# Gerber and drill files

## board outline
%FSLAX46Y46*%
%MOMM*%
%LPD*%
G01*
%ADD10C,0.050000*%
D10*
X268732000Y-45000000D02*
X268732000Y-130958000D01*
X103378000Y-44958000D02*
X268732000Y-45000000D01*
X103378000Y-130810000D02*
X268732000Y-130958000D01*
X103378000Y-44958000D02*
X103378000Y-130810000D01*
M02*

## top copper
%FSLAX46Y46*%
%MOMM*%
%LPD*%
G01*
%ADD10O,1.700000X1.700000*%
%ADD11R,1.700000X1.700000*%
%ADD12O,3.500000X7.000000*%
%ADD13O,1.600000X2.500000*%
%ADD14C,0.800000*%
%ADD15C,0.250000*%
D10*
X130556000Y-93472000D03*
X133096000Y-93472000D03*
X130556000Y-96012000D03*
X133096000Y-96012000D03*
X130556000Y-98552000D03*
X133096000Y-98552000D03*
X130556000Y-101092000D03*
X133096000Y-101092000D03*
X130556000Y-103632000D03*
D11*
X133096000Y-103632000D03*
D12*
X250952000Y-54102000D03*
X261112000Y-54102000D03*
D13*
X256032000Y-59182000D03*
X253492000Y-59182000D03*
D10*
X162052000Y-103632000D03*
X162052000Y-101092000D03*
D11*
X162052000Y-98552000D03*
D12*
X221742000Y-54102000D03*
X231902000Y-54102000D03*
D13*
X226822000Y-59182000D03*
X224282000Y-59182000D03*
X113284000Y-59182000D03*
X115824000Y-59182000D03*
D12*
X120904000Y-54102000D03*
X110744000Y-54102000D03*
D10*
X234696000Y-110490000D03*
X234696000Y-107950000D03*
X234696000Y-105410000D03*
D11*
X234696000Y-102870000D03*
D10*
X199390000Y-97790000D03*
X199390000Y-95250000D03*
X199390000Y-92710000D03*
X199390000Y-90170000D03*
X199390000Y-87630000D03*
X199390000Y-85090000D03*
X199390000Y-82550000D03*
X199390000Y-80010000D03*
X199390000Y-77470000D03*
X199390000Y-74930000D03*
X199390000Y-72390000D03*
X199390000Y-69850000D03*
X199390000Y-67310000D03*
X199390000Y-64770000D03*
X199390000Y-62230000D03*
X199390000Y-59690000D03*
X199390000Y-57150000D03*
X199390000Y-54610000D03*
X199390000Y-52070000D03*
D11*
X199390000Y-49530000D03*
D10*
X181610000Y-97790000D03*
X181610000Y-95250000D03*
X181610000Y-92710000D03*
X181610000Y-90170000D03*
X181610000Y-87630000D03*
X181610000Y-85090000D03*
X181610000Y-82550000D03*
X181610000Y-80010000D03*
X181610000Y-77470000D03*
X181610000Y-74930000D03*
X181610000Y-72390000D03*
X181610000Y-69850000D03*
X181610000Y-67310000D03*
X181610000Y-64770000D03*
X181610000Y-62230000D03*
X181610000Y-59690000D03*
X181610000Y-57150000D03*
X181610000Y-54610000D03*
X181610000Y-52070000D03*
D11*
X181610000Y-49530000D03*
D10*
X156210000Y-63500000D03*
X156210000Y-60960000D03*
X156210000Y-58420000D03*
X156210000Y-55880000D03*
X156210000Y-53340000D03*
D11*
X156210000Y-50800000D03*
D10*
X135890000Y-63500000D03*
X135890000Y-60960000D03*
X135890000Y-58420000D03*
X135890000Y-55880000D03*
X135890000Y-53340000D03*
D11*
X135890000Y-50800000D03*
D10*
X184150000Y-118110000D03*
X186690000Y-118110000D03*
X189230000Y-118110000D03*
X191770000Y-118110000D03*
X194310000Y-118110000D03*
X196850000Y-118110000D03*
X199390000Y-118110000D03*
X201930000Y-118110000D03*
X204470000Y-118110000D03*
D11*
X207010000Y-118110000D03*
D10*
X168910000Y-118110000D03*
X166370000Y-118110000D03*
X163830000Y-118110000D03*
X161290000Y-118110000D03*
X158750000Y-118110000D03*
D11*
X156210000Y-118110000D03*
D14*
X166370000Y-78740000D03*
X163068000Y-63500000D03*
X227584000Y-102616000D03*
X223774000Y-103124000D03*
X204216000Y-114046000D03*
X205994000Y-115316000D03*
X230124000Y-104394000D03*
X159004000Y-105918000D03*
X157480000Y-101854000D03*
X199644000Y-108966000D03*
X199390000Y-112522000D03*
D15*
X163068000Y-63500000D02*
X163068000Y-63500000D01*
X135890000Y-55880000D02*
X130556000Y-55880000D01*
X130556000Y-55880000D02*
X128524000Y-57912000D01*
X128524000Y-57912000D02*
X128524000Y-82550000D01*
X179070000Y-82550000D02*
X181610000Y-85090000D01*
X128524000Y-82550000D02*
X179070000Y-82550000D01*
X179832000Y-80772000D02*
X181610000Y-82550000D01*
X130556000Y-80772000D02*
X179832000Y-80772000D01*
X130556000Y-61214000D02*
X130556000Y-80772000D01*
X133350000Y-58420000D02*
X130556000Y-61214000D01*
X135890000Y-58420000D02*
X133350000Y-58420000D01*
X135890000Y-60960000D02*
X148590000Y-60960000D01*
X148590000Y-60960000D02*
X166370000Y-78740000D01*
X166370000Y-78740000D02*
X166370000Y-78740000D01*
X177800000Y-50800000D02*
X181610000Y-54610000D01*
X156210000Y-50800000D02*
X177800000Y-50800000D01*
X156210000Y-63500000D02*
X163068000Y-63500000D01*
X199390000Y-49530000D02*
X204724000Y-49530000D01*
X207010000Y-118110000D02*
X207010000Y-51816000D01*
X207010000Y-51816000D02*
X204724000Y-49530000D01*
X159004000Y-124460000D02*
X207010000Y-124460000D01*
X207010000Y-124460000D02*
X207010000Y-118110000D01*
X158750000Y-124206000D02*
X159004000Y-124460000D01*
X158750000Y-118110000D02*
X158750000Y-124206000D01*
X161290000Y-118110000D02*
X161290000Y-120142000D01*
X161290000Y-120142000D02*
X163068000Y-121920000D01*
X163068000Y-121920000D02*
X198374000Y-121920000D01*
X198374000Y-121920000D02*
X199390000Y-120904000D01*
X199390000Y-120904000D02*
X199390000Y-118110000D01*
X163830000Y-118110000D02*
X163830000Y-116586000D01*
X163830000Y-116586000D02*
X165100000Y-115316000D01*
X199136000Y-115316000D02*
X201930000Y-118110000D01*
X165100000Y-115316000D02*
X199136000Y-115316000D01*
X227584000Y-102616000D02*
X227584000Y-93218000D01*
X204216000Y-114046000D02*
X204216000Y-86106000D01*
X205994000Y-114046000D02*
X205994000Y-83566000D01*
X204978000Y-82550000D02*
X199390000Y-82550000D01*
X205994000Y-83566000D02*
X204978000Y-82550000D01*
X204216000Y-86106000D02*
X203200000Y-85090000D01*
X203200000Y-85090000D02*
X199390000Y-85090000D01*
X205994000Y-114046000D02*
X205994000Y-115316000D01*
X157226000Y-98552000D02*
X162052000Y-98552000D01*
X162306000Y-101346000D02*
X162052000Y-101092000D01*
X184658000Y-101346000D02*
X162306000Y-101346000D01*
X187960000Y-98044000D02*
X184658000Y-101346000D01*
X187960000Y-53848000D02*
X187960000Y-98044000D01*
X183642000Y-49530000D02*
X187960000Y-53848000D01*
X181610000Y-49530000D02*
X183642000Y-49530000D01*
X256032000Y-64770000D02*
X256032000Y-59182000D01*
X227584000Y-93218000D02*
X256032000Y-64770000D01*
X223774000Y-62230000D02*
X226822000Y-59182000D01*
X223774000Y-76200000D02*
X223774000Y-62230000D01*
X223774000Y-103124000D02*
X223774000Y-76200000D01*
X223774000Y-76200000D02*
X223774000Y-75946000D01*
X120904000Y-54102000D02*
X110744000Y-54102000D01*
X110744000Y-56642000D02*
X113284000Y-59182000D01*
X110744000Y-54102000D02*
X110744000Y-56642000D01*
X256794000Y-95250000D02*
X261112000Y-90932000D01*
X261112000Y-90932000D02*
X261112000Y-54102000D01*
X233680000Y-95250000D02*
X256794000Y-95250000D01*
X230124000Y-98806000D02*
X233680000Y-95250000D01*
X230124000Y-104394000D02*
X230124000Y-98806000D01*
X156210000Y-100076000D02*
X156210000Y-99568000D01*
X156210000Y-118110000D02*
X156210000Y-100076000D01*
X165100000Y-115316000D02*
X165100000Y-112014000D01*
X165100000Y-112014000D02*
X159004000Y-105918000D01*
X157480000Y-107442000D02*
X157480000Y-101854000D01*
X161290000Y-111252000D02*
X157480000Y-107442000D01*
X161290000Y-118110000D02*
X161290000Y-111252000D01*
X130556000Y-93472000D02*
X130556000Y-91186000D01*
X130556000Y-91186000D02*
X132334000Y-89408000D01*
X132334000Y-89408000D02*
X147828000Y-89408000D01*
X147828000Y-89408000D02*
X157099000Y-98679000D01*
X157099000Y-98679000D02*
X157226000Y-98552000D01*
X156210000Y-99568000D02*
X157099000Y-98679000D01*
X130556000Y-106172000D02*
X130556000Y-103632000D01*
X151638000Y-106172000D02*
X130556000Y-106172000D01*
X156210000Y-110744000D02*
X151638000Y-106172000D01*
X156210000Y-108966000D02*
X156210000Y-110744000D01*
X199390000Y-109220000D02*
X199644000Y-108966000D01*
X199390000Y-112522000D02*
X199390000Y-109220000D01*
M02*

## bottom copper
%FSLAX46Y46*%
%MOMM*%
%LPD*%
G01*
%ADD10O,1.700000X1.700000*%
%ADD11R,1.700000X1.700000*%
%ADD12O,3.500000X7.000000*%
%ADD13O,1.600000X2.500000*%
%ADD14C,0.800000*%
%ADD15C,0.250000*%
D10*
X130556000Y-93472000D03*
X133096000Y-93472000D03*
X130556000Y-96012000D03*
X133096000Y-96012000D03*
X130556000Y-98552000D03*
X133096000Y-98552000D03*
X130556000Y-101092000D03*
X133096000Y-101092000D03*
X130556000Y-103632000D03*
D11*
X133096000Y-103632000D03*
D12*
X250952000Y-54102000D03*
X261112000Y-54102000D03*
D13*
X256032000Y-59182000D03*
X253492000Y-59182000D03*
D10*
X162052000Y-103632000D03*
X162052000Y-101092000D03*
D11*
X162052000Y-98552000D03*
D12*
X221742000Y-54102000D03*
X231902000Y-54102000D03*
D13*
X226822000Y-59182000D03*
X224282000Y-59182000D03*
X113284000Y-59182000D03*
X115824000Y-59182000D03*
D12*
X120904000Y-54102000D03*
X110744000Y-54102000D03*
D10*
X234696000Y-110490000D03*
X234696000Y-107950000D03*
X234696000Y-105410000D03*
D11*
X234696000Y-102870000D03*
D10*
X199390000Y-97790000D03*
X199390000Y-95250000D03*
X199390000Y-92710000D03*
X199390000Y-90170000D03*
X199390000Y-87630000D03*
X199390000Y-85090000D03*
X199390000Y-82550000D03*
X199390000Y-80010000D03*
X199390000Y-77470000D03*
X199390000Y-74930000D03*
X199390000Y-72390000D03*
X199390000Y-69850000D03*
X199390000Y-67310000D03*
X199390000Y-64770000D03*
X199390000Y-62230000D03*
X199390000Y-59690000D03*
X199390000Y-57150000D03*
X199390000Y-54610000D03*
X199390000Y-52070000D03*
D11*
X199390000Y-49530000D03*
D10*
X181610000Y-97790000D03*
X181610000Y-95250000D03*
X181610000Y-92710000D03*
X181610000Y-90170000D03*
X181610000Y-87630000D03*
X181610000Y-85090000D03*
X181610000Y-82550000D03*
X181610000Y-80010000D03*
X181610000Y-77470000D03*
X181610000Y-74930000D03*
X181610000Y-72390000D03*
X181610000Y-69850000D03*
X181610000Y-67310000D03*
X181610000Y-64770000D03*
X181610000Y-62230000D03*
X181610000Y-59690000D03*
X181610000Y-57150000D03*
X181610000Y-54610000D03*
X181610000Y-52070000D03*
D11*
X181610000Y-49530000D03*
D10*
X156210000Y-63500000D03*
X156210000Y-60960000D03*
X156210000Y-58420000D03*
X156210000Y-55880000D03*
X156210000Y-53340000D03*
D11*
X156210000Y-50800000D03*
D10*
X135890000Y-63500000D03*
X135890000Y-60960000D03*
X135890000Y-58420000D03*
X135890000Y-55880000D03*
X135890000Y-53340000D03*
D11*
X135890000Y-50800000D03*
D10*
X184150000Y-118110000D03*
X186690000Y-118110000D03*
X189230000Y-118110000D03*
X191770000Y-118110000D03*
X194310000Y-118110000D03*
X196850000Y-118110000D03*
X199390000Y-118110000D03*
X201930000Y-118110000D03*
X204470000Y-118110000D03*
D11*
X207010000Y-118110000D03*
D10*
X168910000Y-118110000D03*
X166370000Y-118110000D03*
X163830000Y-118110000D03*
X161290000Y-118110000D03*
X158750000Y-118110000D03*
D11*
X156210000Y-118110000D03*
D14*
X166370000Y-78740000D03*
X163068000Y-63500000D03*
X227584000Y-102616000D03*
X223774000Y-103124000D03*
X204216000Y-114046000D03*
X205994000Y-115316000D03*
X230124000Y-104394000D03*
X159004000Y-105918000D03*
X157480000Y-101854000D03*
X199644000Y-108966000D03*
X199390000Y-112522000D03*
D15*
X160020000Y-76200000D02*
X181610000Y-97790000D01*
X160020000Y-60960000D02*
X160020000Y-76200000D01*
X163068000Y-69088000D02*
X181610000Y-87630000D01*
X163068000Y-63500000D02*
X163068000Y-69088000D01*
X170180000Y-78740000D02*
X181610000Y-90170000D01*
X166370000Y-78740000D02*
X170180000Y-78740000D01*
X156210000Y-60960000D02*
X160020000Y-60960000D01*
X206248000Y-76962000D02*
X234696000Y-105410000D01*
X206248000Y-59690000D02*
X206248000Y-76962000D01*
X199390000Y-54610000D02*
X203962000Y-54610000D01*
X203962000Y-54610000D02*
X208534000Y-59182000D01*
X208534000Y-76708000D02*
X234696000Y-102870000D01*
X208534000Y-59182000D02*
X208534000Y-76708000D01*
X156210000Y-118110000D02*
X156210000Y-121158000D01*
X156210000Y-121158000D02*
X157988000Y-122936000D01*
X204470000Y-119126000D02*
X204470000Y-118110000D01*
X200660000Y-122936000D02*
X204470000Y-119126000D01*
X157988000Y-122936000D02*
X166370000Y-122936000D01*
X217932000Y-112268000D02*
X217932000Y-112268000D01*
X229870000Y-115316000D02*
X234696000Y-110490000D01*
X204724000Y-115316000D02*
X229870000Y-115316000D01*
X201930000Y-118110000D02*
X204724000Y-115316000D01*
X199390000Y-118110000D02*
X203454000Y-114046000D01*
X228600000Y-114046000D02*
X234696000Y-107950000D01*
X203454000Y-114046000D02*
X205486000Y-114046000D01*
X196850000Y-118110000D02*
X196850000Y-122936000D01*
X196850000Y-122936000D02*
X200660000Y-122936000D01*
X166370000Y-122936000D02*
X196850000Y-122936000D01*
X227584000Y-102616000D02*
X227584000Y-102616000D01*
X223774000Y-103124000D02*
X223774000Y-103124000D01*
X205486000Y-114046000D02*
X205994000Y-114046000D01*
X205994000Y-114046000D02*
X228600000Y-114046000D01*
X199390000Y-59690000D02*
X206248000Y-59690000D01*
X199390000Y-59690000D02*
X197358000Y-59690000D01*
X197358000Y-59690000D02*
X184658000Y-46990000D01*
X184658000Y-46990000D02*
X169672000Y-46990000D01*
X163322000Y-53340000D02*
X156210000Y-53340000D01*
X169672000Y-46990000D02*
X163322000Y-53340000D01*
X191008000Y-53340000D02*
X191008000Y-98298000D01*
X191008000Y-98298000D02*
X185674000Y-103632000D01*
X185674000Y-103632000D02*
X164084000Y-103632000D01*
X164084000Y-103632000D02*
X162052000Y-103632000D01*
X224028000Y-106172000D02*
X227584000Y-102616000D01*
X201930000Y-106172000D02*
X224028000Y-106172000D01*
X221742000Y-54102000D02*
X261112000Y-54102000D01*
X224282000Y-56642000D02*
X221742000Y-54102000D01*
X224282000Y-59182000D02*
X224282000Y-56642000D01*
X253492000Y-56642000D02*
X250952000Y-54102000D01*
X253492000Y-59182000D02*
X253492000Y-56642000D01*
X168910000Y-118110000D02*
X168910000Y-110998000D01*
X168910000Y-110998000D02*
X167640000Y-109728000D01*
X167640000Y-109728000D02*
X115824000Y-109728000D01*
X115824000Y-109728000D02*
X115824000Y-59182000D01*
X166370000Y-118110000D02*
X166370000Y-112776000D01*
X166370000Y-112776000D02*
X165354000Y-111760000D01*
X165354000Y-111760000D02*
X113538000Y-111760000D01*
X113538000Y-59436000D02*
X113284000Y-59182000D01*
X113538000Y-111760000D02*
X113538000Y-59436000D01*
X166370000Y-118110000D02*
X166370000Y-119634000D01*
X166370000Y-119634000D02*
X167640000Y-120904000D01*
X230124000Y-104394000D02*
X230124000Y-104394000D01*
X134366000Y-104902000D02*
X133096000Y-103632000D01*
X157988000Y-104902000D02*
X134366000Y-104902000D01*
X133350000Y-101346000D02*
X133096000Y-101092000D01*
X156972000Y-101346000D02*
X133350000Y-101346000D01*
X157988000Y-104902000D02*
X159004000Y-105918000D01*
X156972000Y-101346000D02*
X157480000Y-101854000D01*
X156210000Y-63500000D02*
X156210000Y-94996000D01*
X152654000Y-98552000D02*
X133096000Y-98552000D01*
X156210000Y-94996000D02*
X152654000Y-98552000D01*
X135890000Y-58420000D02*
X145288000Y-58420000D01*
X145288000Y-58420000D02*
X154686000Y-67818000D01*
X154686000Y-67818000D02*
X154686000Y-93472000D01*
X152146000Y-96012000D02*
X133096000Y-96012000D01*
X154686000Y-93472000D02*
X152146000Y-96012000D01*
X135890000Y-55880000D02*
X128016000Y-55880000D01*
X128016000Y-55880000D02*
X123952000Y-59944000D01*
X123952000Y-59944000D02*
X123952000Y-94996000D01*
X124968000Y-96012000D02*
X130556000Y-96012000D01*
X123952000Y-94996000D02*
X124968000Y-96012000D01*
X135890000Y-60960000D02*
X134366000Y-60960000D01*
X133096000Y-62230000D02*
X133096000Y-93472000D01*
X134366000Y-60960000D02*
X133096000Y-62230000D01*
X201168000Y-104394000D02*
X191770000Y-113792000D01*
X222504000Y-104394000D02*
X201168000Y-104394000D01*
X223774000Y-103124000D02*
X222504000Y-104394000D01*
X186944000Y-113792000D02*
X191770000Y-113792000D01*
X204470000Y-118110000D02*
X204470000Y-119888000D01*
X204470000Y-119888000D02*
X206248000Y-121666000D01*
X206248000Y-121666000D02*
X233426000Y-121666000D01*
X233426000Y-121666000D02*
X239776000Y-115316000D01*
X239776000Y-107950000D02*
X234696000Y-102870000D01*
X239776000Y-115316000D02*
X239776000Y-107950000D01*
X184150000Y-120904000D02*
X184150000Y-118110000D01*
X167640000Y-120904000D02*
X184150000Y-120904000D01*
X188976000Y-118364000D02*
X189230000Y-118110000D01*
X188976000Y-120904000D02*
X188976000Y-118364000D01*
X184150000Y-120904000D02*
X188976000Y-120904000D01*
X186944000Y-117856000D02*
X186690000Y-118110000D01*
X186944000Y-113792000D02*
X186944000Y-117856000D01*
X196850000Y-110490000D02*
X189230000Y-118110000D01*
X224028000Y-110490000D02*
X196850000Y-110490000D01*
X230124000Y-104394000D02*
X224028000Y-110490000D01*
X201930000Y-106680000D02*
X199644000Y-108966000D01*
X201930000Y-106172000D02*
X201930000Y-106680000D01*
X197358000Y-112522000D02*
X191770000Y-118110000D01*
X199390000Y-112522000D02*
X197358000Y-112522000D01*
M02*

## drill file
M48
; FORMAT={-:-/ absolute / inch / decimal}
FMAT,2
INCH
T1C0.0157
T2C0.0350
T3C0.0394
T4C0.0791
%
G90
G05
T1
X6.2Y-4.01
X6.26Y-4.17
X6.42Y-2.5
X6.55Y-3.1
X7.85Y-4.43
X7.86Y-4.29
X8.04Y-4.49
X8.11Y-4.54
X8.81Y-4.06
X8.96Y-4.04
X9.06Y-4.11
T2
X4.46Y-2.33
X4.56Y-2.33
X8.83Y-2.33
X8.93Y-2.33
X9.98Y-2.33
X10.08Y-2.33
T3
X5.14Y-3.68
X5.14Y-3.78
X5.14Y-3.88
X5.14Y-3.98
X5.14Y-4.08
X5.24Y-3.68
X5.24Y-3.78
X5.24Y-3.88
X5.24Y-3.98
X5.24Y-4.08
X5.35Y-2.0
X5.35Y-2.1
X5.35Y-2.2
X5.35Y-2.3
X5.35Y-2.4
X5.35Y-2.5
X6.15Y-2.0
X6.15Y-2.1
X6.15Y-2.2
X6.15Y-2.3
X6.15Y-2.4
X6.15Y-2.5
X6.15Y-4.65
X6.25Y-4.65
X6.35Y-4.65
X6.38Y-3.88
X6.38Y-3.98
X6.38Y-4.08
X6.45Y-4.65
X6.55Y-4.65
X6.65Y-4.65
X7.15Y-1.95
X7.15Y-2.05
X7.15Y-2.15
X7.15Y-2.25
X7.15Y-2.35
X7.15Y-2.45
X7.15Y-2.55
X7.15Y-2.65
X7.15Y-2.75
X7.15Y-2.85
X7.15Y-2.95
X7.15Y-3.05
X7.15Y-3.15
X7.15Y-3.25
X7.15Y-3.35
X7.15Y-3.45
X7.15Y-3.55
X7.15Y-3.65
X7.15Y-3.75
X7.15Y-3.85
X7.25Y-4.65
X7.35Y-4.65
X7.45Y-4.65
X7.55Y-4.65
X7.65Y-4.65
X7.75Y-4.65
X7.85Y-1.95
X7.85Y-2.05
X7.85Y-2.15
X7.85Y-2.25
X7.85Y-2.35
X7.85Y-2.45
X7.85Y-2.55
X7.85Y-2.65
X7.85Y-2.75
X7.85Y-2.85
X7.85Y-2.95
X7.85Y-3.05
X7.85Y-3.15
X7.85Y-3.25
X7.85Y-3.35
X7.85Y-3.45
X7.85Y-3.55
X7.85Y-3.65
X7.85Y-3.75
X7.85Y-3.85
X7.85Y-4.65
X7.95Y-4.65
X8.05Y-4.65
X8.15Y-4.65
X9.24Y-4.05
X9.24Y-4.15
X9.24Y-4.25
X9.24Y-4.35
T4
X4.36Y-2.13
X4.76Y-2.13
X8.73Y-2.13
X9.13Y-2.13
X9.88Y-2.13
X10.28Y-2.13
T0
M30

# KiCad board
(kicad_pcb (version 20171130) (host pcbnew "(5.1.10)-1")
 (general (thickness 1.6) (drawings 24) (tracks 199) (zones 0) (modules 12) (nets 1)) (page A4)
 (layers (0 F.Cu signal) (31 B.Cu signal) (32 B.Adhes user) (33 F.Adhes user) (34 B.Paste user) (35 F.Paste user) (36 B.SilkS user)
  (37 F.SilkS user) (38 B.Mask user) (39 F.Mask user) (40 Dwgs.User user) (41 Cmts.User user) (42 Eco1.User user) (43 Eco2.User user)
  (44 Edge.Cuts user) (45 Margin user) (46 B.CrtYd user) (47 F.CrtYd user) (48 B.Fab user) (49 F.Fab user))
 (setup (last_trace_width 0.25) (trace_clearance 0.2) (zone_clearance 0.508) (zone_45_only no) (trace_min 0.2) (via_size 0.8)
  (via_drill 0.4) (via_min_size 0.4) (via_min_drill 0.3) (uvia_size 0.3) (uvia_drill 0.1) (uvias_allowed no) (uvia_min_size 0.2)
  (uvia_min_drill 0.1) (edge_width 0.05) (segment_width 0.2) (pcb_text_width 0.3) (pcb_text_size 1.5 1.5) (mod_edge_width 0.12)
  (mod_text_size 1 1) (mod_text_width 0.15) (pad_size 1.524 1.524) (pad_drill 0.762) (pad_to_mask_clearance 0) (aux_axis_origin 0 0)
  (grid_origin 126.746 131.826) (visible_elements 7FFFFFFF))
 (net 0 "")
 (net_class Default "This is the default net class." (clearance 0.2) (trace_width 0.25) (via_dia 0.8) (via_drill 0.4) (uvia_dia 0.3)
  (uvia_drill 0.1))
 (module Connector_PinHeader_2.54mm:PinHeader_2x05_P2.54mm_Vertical (layer F.Cu) (at 133.096 103.632 180)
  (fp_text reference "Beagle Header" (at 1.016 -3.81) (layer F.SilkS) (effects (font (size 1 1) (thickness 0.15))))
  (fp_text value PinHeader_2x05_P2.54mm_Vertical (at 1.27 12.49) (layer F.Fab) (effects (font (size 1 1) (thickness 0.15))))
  (pad 10 thru_hole oval (at 2.54 10.16 180) (size 1.7 1.7) (drill 1) (layers *.Cu *.Mask))
  (pad 9 thru_hole oval (at 0 10.16 180) (size 1.7 1.7) (drill 1) (layers *.Cu *.Mask))
  (pad 8 thru_hole oval (at 2.54 7.62 180) (size 1.7 1.7) (drill 1) (layers *.Cu *.Mask))
  (pad 7 thru_hole oval (at 0 7.62 180) (size 1.7 1.7) (drill 1) (layers *.Cu *.Mask))
  (pad 6 thru_hole oval (at 2.54 5.08 180) (size 1.7 1.7) (drill 1) (layers *.Cu *.Mask))
  (pad 5 thru_hole oval (at 0 5.08 180) (size 1.7 1.7) (drill 1) (layers *.Cu *.Mask))
  (pad 4 thru_hole oval (at 2.54 2.54 180) (size 1.7 1.7) (drill 1) (layers *.Cu *.Mask))
  (pad 3 thru_hole oval (at 0 2.54 180) (size 1.7 1.7) (drill 1) (layers *.Cu *.Mask))
  (pad 2 thru_hole oval (at 2.54 0 180) (size 1.7 1.7) (drill 1) (layers *.Cu *.Mask))
  (pad 1 thru_hole rect (at 0 0 180) (size 1.7 1.7) (drill 1) (layers *.Cu *.Mask)))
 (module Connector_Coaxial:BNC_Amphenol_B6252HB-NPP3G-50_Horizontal (layer F.Cu) (at 256.032 59.182)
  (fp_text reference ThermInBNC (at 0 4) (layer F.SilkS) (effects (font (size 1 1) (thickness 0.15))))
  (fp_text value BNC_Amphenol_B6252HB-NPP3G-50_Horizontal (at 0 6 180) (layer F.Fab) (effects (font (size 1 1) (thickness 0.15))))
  (pad 2 thru_hole oval (at -5.08 -5.08) (size 3.5 7) (drill 2.01) (layers *.Cu *.Mask))
  (pad 2 thru_hole oval (at 5.08 -5.08) (size 3.5 7) (drill 2.01) (layers *.Cu *.Mask))
  (pad 1 thru_hole oval (at 0 0) (size 1.6 2.5) (drill 0.89) (layers *.Cu *.Mask))
  (pad 2 thru_hole oval (at -2.54 0) (size 1.6 2.5) (drill 0.89) (layers *.Cu *.Mask)))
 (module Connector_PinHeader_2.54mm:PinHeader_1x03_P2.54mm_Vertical (layer F.Cu) (at 162.052 98.552)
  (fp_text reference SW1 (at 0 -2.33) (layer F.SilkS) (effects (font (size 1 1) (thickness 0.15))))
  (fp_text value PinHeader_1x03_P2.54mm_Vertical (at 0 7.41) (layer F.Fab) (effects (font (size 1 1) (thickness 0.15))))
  (pad 3 thru_hole oval (at 0 5.08) (size 1.7 1.7) (drill 1) (layers *.Cu *.Mask))
  (pad 2 thru_hole oval (at 0 2.54) (size 1.7 1.7) (drill 1) (layers *.Cu *.Mask))
  (pad 1 thru_hole rect (at 0 0) (size 1.7 1.7) (drill 1) (layers *.Cu *.Mask)))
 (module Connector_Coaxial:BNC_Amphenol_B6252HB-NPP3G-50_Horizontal (layer F.Cu) (at 226.822 59.182)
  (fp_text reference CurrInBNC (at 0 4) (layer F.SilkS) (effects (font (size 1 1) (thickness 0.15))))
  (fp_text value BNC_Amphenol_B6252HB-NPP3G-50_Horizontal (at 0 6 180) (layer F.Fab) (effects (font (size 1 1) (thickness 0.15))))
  (pad 2 thru_hole oval (at -5.08 -5.08) (size 3.5 7) (drill 2.01) (layers *.Cu *.Mask))
  (pad 2 thru_hole oval (at 5.08 -5.08) (size 3.5 7) (drill 2.01) (layers *.Cu *.Mask))
  (pad 1 thru_hole oval (at 0 0) (size 1.6 2.5) (drill 0.89) (layers *.Cu *.Mask))
  (pad 2 thru_hole oval (at -2.54 0) (size 1.6 2.5) (drill 0.89) (layers *.Cu *.Mask)))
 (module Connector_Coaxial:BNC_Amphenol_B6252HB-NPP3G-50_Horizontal (layer F.Cu) (at 115.824 59.182)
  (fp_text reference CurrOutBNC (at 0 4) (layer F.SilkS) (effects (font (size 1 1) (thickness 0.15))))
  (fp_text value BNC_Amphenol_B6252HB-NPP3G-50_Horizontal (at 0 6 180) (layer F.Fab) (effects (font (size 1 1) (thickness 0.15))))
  (pad 2 thru_hole oval (at -2.54 0) (size 1.6 2.5) (drill 0.89) (layers *.Cu *.Mask))
  (pad 1 thru_hole oval (at 0 0) (size 1.6 2.5) (drill 0.89) (layers *.Cu *.Mask))
  (pad 2 thru_hole oval (at 5.08 -5.08) (size 3.5 7) (drill 2.01) (layers *.Cu *.Mask))
  (pad 2 thru_hole oval (at -5.08 -5.08) (size 3.5 7) (drill 2.01) (layers *.Cu *.Mask)))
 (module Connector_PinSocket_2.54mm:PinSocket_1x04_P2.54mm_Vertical (layer F.Cu) (at 234.696 102.87)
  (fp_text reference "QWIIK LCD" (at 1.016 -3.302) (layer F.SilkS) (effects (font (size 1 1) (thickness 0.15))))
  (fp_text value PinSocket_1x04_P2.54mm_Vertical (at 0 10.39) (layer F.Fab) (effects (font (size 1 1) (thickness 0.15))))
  (pad 4 thru_hole oval (at 0 7.62) (size 1.7 1.7) (drill 1) (layers *.Cu *.Mask))
  (pad 3 thru_hole oval (at 0 5.08) (size 1.7 1.7) (drill 1) (layers *.Cu *.Mask))
  (pad 2 thru_hole oval (at 0 2.54) (size 1.7 1.7) (drill 1) (layers *.Cu *.Mask))
  (pad 1 thru_hole rect (at 0 0) (size 1.7 1.7) (drill 1) (layers *.Cu *.Mask)))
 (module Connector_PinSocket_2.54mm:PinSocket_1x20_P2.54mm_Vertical (layer F.Cu) (at 199.39 49.53)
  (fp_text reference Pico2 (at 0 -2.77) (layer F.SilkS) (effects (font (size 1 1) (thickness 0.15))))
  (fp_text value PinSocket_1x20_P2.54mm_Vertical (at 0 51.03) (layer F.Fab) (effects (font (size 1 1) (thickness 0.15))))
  (pad 20 thru_hole oval (at 0 48.26) (size 1.7 1.7) (drill 1) (layers *.Cu *.Mask))
  (pad 19 thru_hole oval (at 0 45.72) (size 1.7 1.7) (drill 1) (layers *.Cu *.Mask))
  (pad 18 thru_hole oval (at 0 43.18) (size 1.7 1.7) (drill 1) (layers *.Cu *.Mask))
  (pad 17 thru_hole oval (at 0 40.64) (size 1.7 1.7) (drill 1) (layers *.Cu *.Mask))
  (pad 16 thru_hole oval (at 0 38.1) (size 1.7 1.7) (drill 1) (layers *.Cu *.Mask))
  (pad 15 thru_hole oval (at 0 35.56) (size 1.7 1.7) (drill 1) (layers *.Cu *.Mask))
  (pad 14 thru_hole oval (at 0 33.02) (size 1.7 1.7) (drill 1) (layers *.Cu *.Mask))
  (pad 13 thru_hole oval (at 0 30.48) (size 1.7 1.7) (drill 1) (layers *.Cu *.Mask))
  (pad 12 thru_hole oval (at 0 27.94) (size 1.7 1.7) (drill 1) (layers *.Cu *.Mask))
  (pad 11 thru_hole oval (at 0 25.4) (size 1.7 1.7) (drill 1) (layers *.Cu *.Mask))
  (pad 10 thru_hole oval (at 0 22.86) (size 1.7 1.7) (drill 1) (layers *.Cu *.Mask))
  (pad 9 thru_hole oval (at 0 20.32) (size 1.7 1.7) (drill 1) (layers *.Cu *.Mask))
  (pad 8 thru_hole oval (at 0 17.78) (size 1.7 1.7) (drill 1) (layers *.Cu *.Mask))
  (pad 7 thru_hole oval (at 0 15.24) (size 1.7 1.7) (drill 1) (layers *.Cu *.Mask))
  (pad 6 thru_hole oval (at 0 12.7) (size 1.7 1.7) (drill 1) (layers *.Cu *.Mask))
  (pad 5 thru_hole oval (at 0 10.16) (size 1.7 1.7) (drill 1) (layers *.Cu *.Mask))
  (pad 4 thru_hole oval (at 0 7.62) (size 1.7 1.7) (drill 1) (layers *.Cu *.Mask))
  (pad 3 thru_hole oval (at 0 5.08) (size 1.7 1.7) (drill 1) (layers *.Cu *.Mask))
  (pad 2 thru_hole oval (at 0 2.54) (size 1.7 1.7) (drill 1) (layers *.Cu *.Mask))
  (pad 1 thru_hole rect (at 0 0) (size 1.7 1.7) (drill 1) (layers *.Cu *.Mask)))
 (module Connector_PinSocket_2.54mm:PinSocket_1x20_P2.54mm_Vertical (layer F.Cu) (at 181.61 49.53)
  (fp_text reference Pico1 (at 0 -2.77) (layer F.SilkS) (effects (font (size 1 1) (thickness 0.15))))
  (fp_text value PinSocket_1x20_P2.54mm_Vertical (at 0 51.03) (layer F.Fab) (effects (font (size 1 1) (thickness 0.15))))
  (pad 20 thru_hole oval (at 0 48.26) (size 1.7 1.7) (drill 1) (layers *.Cu *.Mask))
  (pad 19 thru_hole oval (at 0 45.72) (size 1.7 1.7) (drill 1) (layers *.Cu *.Mask))
  (pad 18 thru_hole oval (at 0 43.18) (size 1.7 1.7) (drill 1) (layers *.Cu *.Mask))
  (pad 17 thru_hole oval (at 0 40.64) (size 1.7 1.7) (drill 1) (layers *.Cu *.Mask))
  (pad 16 thru_hole oval (at 0 38.1) (size 1.7 1.7) (drill 1) (layers *.Cu *.Mask))
  (pad 15 thru_hole oval (at 0 35.56) (size 1.7 1.7) (drill 1) (layers *.Cu *.Mask))
  (pad 14 thru_hole oval (at 0 33.02) (size 1.7 1.7) (drill 1) (layers *.Cu *.Mask))
  (pad 13 thru_hole oval (at 0 30.48) (size 1.7 1.7) (drill 1) (layers *.Cu *.Mask))
  (pad 12 thru_hole oval (at 0 27.94) (size 1.7 1.7) (drill 1) (layers *.Cu *.Mask))
  (pad 11 thru_hole oval (at 0 25.4) (size 1.7 1.7) (drill 1) (layers *.Cu *.Mask))
  (pad 10 thru_hole oval (at 0 22.86) (size 1.7 1.7) (drill 1) (layers *.Cu *.Mask))
  (pad 9 thru_hole oval (at 0 20.32) (size 1.7 1.7) (drill 1) (layers *.Cu *.Mask))
  (pad 8 thru_hole oval (at 0 17.78) (size 1.7 1.7) (drill 1) (layers *.Cu *.Mask))
  (pad 7 thru_hole oval (at 0 15.24) (size 1.7 1.7) (drill 1) (layers *.Cu *.Mask))
  (pad 6 thru_hole oval (at 0 12.7) (size 1.7 1.7) (drill 1) (layers *.Cu *.Mask))
  (pad 5 thru_hole oval (at 0 10.16) (size 1.7 1.7) (drill 1) (layers *.Cu *.Mask))
  (pad 4 thru_hole oval (at 0 7.62) (size 1.7 1.7) (drill 1) (layers *.Cu *.Mask))
  (pad 3 thru_hole oval (at 0 5.08) (size 1.7 1.7) (drill 1) (layers *.Cu *.Mask))
  (pad 2 thru_hole oval (at 0 2.54) (size 1.7 1.7) (drill 1) (layers *.Cu *.Mask))
  (pad 1 thru_hole rect (at 0 0) (size 1.7 1.7) (drill 1) (layers *.Cu *.Mask)))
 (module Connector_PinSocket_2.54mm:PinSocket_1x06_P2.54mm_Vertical (layer F.Cu) (at 156.21 50.8)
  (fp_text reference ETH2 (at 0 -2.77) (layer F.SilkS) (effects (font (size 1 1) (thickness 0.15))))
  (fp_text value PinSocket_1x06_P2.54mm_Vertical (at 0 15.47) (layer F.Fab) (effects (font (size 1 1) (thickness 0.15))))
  (pad 6 thru_hole oval (at 0 12.7) (size 1.7 1.7) (drill 1) (layers *.Cu *.Mask))
  (pad 5 thru_hole oval (at 0 10.16) (size 1.7 1.7) (drill 1) (layers *.Cu *.Mask))
  (pad 4 thru_hole oval (at 0 7.62) (size 1.7 1.7) (drill 1) (layers *.Cu *.Mask))
  (pad 3 thru_hole oval (at 0 5.08) (size 1.7 1.7) (drill 1) (layers *.Cu *.Mask))
  (pad 2 thru_hole oval (at 0 2.54) (size 1.7 1.7) (drill 1) (layers *.Cu *.Mask))
  (pad 1 thru_hole rect (at 0 0) (size 1.7 1.7) (drill 1) (layers *.Cu *.Mask)))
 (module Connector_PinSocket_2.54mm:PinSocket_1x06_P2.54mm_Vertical (layer F.Cu) (at 135.89 50.8)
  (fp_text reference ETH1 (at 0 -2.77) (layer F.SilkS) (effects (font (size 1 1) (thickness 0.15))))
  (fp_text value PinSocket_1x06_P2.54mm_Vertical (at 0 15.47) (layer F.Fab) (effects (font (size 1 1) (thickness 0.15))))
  (pad 6 thru_hole oval (at 0 12.7) (size 1.7 1.7) (drill 1) (layers *.Cu *.Mask))
  (pad 5 thru_hole oval (at 0 10.16) (size 1.7 1.7) (drill 1) (layers *.Cu *.Mask))
  (pad 4 thru_hole oval (at 0 7.62) (size 1.7 1.7) (drill 1) (layers *.Cu *.Mask))
  (pad 3 thru_hole oval (at 0 5.08) (size 1.7 1.7) (drill 1) (layers *.Cu *.Mask))
  (pad 2 thru_hole oval (at 0 2.54) (size 1.7 1.7) (drill 1) (layers *.Cu *.Mask))
  (pad 1 thru_hole rect (at 0 0) (size 1.7 1.7) (drill 1) (layers *.Cu *.Mask)))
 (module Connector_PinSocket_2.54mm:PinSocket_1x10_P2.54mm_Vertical (layer F.Cu) (at 207.01 118.11 270)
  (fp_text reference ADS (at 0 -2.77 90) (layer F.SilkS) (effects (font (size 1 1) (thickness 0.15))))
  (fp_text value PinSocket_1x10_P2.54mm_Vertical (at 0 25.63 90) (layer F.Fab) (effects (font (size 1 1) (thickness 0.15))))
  (pad 10 thru_hole oval (at 0 22.86 270) (size 1.7 1.7) (drill 1) (layers *.Cu *.Mask))
  (pad 9 thru_hole oval (at 0 20.32 270) (size 1.7 1.7) (drill 1) (layers *.Cu *.Mask))
  (pad 8 thru_hole oval (at 0 17.78 270) (size 1.7 1.7) (drill 1) (layers *.Cu *.Mask))
  (pad 7 thru_hole oval (at 0 15.24 270) (size 1.7 1.7) (drill 1) (layers *.Cu *.Mask))
  (pad 6 thru_hole oval (at 0 12.7 270) (size 1.7 1.7) (drill 1) (layers *.Cu *.Mask))
  (pad 5 thru_hole oval (at 0 10.16 270) (size 1.7 1.7) (drill 1) (layers *.Cu *.Mask))
  (pad 4 thru_hole oval (at 0 7.62 270) (size 1.7 1.7) (drill 1) (layers *.Cu *.Mask))
  (pad 3 thru_hole oval (at 0 5.08 270) (size 1.7 1.7) (drill 1) (layers *.Cu *.Mask))
  (pad 2 thru_hole oval (at 0 2.54 270) (size 1.7 1.7) (drill 1) (layers *.Cu *.Mask))
  (pad 1 thru_hole rect (at 0 0 270) (size 1.7 1.7) (drill 1) (layers *.Cu *.Mask)))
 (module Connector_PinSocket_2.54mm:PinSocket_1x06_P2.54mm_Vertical (layer F.Cu) (at 156.21 118.11 90)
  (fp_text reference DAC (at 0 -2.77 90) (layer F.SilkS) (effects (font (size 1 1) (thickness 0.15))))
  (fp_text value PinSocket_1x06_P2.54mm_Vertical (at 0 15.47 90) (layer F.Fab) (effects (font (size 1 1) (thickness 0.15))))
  (pad 6 thru_hole oval (at 0 12.7 90) (size 1.7 1.7) (drill 1) (layers *.Cu *.Mask))
  (pad 5 thru_hole oval (at 0 10.16 90) (size 1.7 1.7) (drill 1) (layers *.Cu *.Mask))
  (pad 4 thru_hole oval (at 0 7.62 90) (size 1.7 1.7) (drill 1) (layers *.Cu *.Mask))
  (pad 3 thru_hole oval (at 0 5.08 90) (size 1.7 1.7) (drill 1) (layers *.Cu *.Mask))
  (pad 2 thru_hole oval (at 0 2.54 90) (size 1.7 1.7) (drill 1) (layers *.Cu *.Mask))
  (pad 1 thru_hole rect (at 0 0 90) (size 1.7 1.7) (drill 1) (layers *.Cu *.Mask)))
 (gr_line (start 268.732 45) (end 268.732 130.958) (layer Edge.Cuts) (width 0.05))
 (gr_line (start 103.378 44.958) (end 268.732 45) (layer Edge.Cuts) (width 0.05))
 (gr_line (start 103.378 130.81) (end 268.732 130.958) (layer Edge.Cuts) (width 0.05))
 (gr_line (start 103.378 44.958) (end 103.378 130.81) (layer Edge.Cuts) (width 0.05))
 (segment (start 160.02 76.2) (end 181.61 97.79) (width 0.25) (layer B.Cu) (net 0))
 (segment (start 160.02 60.96) (end 160.02 76.2) (width 0.25) (layer B.Cu) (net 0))
 (segment (start 163.068 63.5) (end 163.068 63.5) (width 0.25) (layer F.Cu) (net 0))
 (segment (start 163.068 69.088) (end 181.61 87.63) (width 0.25) (layer B.Cu) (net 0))
 (segment (start 163.068 63.5) (end 163.068 69.088) (width 0.25) (layer B.Cu) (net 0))
 (segment (start 135.89 55.88) (end 130.556 55.88) (width 0.25) (layer F.Cu) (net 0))
 (segment (start 130.556 55.88) (end 128.524 57.912) (width 0.25) (layer F.Cu) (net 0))
 (segment (start 128.524 57.912) (end 128.524 82.55) (width 0.25) (layer F.Cu) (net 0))
 (segment (start 179.07 82.55) (end 181.61 85.09) (width 0.25) (layer F.Cu) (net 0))
 (segment (start 128.524 82.55) (end 179.07 82.55) (width 0.25) (layer F.Cu) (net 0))
 (segment (start 179.832 80.772) (end 181.61 82.55) (width 0.25) (layer F.Cu) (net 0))
 (segment (start 130.556 80.772) (end 179.832 80.772) (width 0.25) (layer F.Cu) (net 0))
 (segment (start 130.556 61.214) (end 130.556 80.772) (width 0.25) (layer F.Cu) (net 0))
 (segment (start 133.35 58.42) (end 130.556 61.214) (width 0.25) (layer F.Cu) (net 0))
 (segment (start 135.89 58.42) (end 133.35 58.42) (width 0.25) (layer F.Cu) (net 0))
 (segment (start 135.89 60.96) (end 148.59 60.96) (width 0.25) (layer F.Cu) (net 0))
 (segment (start 148.59 60.96) (end 166.37 78.74) (width 0.25) (layer F.Cu) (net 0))
 (segment (start 166.37 78.74) (end 166.37 78.74) (width 0.25) (layer F.Cu) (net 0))
 (via (at 166.37 78.74) (size 0.8) (drill 0.4) (layers F.Cu B.Cu) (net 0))
 (segment (start 170.18 78.74) (end 181.61 90.17) (width 0.25) (layer B.Cu) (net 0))
 (segment (start 166.37 78.74) (end 170.18 78.74) (width 0.25) (layer B.Cu) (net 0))
 (segment (start 177.8 50.8) (end 181.61 54.61) (width 0.25) (layer F.Cu) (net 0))
 (segment (start 156.21 50.8) (end 177.8 50.8) (width 0.25) (layer F.Cu) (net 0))
 (segment (start 156.21 63.5) (end 163.068 63.5) (width 0.25) (layer F.Cu) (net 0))
 (via (at 163.068 63.5) (size 0.8) (drill 0.4) (layers F.Cu B.Cu) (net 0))
 (segment (start 156.21 60.96) (end 160.02 60.96) (width 0.25) (layer B.Cu) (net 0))
 (segment (start 206.248 76.962) (end 234.696 105.41) (width 0.25) (layer B.Cu) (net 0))
 (segment (start 206.248 59.69) (end 206.248 76.962) (width 0.25) (layer B.Cu) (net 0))
 (segment (start 199.39 54.61) (end 203.962 54.61) (width 0.25) (layer B.Cu) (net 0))
 (segment (start 203.962 54.61) (end 208.534 59.182) (width 0.25) (layer B.Cu) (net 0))
 (segment (start 208.534 76.708) (end 234.696 102.87) (width 0.25) (layer B.Cu) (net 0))
 (segment (start 208.534 59.182) (end 208.534 76.708) (width 0.25) (layer B.Cu) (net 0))
 (segment (start 199.39 49.53) (end 204.724 49.53) (width 0.25) (layer F.Cu) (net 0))
 (segment (start 207.01 118.11) (end 207.01 51.816) (width 0.25) (layer F.Cu) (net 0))
 (segment (start 207.01 51.816) (end 204.724 49.53) (width 0.25) (layer F.Cu) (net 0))
 (segment (start 159.004 124.46) (end 207.01 124.46) (width 0.25) (layer F.Cu) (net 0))
 (segment (start 207.01 124.46) (end 207.01 118.11) (width 0.25) (layer F.Cu) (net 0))
 (segment (start 158.75 124.206) (end 159.004 124.46) (width 0.25) (layer F.Cu) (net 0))
 (segment (start 158.75 118.11) (end 158.75 124.206) (width 0.25) (layer F.Cu) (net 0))
 (segment (start 156.21 118.11) (end 156.21 121.158) (width 0.25) (layer B.Cu) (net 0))
 (segment (start 156.21 121.158) (end 157.988 122.936) (width 0.25) (layer B.Cu) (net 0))
 (segment (start 204.47 119.126) (end 204.47 118.11) (width 0.25) (layer B.Cu) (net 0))
 (segment (start 200.66 122.936) (end 204.47 119.126) (width 0.25) (layer B.Cu) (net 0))
 (segment (start 161.29 118.11) (end 161.29 120.142) (width 0.25) (layer F.Cu) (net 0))
 (segment (start 161.29 120.142) (end 163.068 121.92) (width 0.25) (layer F.Cu) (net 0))
 (segment (start 163.068 121.92) (end 198.374 121.92) (width 0.25) (layer F.Cu) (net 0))
 (segment (start 198.374 121.92) (end 199.39 120.904) (width 0.25) (layer F.Cu) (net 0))
 (segment (start 199.39 120.904) (end 199.39 118.11) (width 0.25) (layer F.Cu) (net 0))
 (segment (start 163.83 118.11) (end 163.83 116.586) (width 0.25) (layer F.Cu) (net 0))
 (segment (start 163.83 116.586) (end 165.1 115.316) (width 0.25) (layer F.Cu) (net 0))
 (segment (start 199.136 115.316) (end 201.93 118.11) (width 0.25) (layer F.Cu) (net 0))
 (segment (start 165.1 115.316) (end 199.136 115.316) (width 0.25) (layer F.Cu) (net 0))
 (segment (start 157.988 122.936) (end 166.37 122.936) (width 0.25) (layer B.Cu) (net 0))
 (segment (start 217.932 112.268) (end 217.932 112.268) (width 0.25) (layer B.Cu) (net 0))
 (segment (start 229.87 115.316) (end 234.696 110.49) (width 0.25) (layer B.Cu) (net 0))
 (segment (start 204.724 115.316) (end 229.87 115.316) (width 0.25) (layer B.Cu) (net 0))
 (segment (start 201.93 118.11) (end 204.724 115.316) (width 0.25) (layer B.Cu) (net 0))
 (segment (start 199.39 118.11) (end 203.454 114.046) (width 0.25) (layer B.Cu) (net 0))
 (segment (start 228.6 114.046) (end 234.696 107.95) (width 0.25) (layer B.Cu) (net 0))
 (segment (start 203.454 114.046) (end 205.486 114.046) (width 0.25) (layer B.Cu) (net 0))
 (segment (start 196.85 118.11) (end 196.85 122.936) (width 0.25) (layer B.Cu) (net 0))
 (segment (start 196.85 122.936) (end 200.66 122.936) (width 0.25) (layer B.Cu) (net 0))
 (segment (start 166.37 122.936) (end 196.85 122.936) (width 0.25) (layer B.Cu) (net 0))
 (segment (start 227.584 102.616) (end 227.584 102.616) (width 0.25) (layer B.Cu) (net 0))
 (via (at 227.584 102.616) (size 0.8) (drill 0.4) (layers F.Cu B.Cu) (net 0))
 (segment (start 227.584 102.616) (end 227.584 93.218) (width 0.25) (layer F.Cu) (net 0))
 (segment (start 223.774 103.124) (end 223.774 103.124) (width 0.25) (layer B.Cu) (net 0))
 (via (at 223.774 103.124) (size 0.8) (drill 0.4) (layers F.Cu B.Cu) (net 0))
 (segment (start 205.486 114.046) (end 205.994 114.046) (width 0.25) (layer B.Cu) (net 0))
 (via (at 204.216 114.046) (size 0.8) (drill 0.4) (layers F.Cu B.Cu) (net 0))
 (segment (start 204.216 114.046) (end 204.216 86.106) (width 0.25) (layer F.Cu) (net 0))
 (segment (start 205.994 114.046) (end 228.6 114.046) (width 0.25) (layer B.Cu) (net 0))
 (via (at 205.994 115.316) (size 0.8) (drill 0.4) (layers F.Cu B.Cu) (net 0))
 (segment (start 205.994 114.046) (end 205.994 83.566) (width 0.25) (layer F.Cu) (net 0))
 (segment (start 204.978 82.55) (end 199.39 82.55) (width 0.25) (layer F.Cu) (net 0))
 (segment (start 205.994 83.566) (end 204.978 82.55) (width 0.25) (layer F.Cu) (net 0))
 (segment (start 204.216 86.106) (end 203.2 85.09) (width 0.25) (layer F.Cu) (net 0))
 (segment (start 203.2 85.09) (end 199.39 85.09) (width 0.25) (layer F.Cu) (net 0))
 (segment (start 205.994 114.046) (end 205.994 115.316) (width 0.25) (layer F.Cu) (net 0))
 (segment (start 199.39 59.69) (end 206.248 59.69) (width 0.25) (layer B.Cu) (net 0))
 (segment (start 199.39 59.69) (end 197.358 59.69) (width 0.25) (layer B.Cu) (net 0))
 (segment (start 197.358 59.69) (end 184.658 46.99) (width 0.25) (layer B.Cu) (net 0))
 (segment (start 184.658 46.99) (end 169.672 46.99) (width 0.25) (layer B.Cu) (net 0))
 (segment (start 163.322 53.34) (end 156.21 53.34) (width 0.25) (layer B.Cu) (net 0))
 (segment (start 169.672 46.99) (end 163.322 53.34) (width 0.25) (layer B.Cu) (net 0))
 (segment (start 191.008 53.34) (end 191.008 98.298) (width 0.25) (layer B.Cu) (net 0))
 (segment (start 191.008 98.298) (end 185.674 103.632) (width 0.25) (layer B.Cu) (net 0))
 (segment (start 185.674 103.632) (end 164.084 103.632) (width 0.25) (layer B.Cu) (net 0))
 (segment (start 157.226 98.552) (end 162.052 98.552) (width 0.25) (layer F.Cu) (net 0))
 (segment (start 162.306 101.346) (end 162.052 101.092) (width 0.25) (layer F.Cu) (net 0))
 (segment (start 184.658 101.346) (end 162.306 101.346) (width 0.25) (layer F.Cu) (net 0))
 (segment (start 187.96 98.044) (end 184.658 101.346) (width 0.25) (layer F.Cu) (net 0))
 (segment (start 187.96 53.848) (end 187.96 98.044) (width 0.25) (layer F.Cu) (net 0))
 (segment (start 183.642 49.53) (end 187.96 53.848) (width 0.25) (layer F.Cu) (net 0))
 (segment (start 181.61 49.53) (end 183.642 49.53) (width 0.25) (layer F.Cu) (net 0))
 (segment (start 164.084 103.632) (end 162.052 103.632) (width 0.25) (layer B.Cu) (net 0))
 (segment (start 256.032 64.77) (end 256.032 59.182) (width 0.25) (layer F.Cu) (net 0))
 (segment (start 227.584 93.218) (end 256.032 64.77) (width 0.25) (layer F.Cu) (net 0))
 (segment (start 223.774 62.23) (end 226.822 59.182) (width 0.25) (layer F.Cu) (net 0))
 (segment (start 223.774 76.2) (end 223.774 62.23) (width 0.25) (layer F.Cu) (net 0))
 (segment (start 223.774 103.124) (end 223.774 76.2) (width 0.25) (layer F.Cu) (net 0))
 (segment (start 223.774 76.2) (end 223.774 75.946) (width 0.25) (layer F.Cu) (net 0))
 (segment (start 224.028 106.172) (end 227.584 102.616) (width 0.25) (layer B.Cu) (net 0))
 (segment (start 201.93 106.172) (end 224.028 106.172) (width 0.25) (layer B.Cu) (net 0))
 (segment (start 221.742 54.102) (end 261.112 54.102) (width 0.25) (layer B.Cu) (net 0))
 (segment (start 224.282 56.642) (end 221.742 54.102) (width 0.25) (layer B.Cu) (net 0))
 (segment (start 224.282 59.182) (end 224.282 56.642) (width 0.25) (layer B.Cu) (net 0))
 (segment (start 253.492 56.642) (end 250.952 54.102) (width 0.25) (layer B.Cu) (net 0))
 (segment (start 253.492 59.182) (end 253.492 56.642) (width 0.25) (layer B.Cu) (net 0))
 (segment (start 168.91 118.11) (end 168.91 110.998) (width 0.25) (layer B.Cu) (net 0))
 (segment (start 168.91 110.998) (end 167.64 109.728) (width 0.25) (layer B.Cu) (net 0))
 (segment (start 167.64 109.728) (end 115.824 109.728) (width 0.25) (layer B.Cu) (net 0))
 (segment (start 115.824 109.728) (end 115.824 59.182) (width 0.25) (layer B.Cu) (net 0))
 (segment (start 120.904 54.102) (end 110.744 54.102) (width 0.25) (layer F.Cu) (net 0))
 (segment (start 110.744 56.642) (end 113.284 59.182) (width 0.25) (layer F.Cu) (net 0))
 (segment (start 110.744 54.102) (end 110.744 56.642) (width 0.25) (layer F.Cu) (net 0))
 (segment (start 166.37 118.11) (end 166.37 112.776) (width 0.25) (layer B.Cu) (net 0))
 (segment (start 166.37 112.776) (end 165.354 111.76) (width 0.25) (layer B.Cu) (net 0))
 (segment (start 165.354 111.76) (end 113.538 111.76) (width 0.25) (layer B.Cu) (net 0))
 (segment (start 113.538 59.436) (end 113.284 59.182) (width 0.25) (layer B.Cu) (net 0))
 (segment (start 113.538 111.76) (end 113.538 59.436) (width 0.25) (layer B.Cu) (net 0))
 (segment (start 166.37 118.11) (end 166.37 119.634) (width 0.25) (layer B.Cu) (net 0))
 (segment (start 166.37 119.634) (end 167.64 120.904) (width 0.25) (layer B.Cu) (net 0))
 (segment (start 230.124 104.394) (end 230.124 104.394) (width 0.25) (layer B.Cu) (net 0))
 (via (at 230.124 104.394) (size 0.8) (drill 0.4) (layers F.Cu B.Cu) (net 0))
 (segment (start 256.794 95.25) (end 261.112 90.932) (width 0.25) (layer F.Cu) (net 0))
 (segment (start 261.112 90.932) (end 261.112 54.102) (width 0.25) (layer F.Cu) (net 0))
 (segment (start 233.68 95.25) (end 256.794 95.25) (width 0.25) (layer F.Cu) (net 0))
 (segment (start 230.124 98.806) (end 233.68 95.25) (width 0.25) (layer F.Cu) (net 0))
 (segment (start 230.124 104.394) (end 230.124 98.806) (width 0.25) (layer F.Cu) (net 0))
 (segment (start 156.21 100.076) (end 156.21 99.568) (width 0.25) (layer F.Cu) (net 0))
 (segment (start 156.21 118.11) (end 156.21 100.076) (width 0.25) (layer F.Cu) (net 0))
 (segment (start 165.1 115.316) (end 165.1 112.014) (width 0.25) (layer F.Cu) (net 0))
 (via (at 159.004 105.918) (size 0.8) (drill 0.4) (layers F.Cu B.Cu) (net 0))
 (segment (start 134.366 104.902) (end 133.096 103.632) (width 0.25) (layer B.Cu) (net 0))
 (segment (start 157.988 104.902) (end 134.366 104.902) (width 0.25) (layer B.Cu) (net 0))
 (via (at 157.48 101.854) (size 0.8) (drill 0.4) (layers F.Cu B.Cu) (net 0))
 (segment (start 133.35 101.346) (end 133.096 101.092) (width 0.25) (layer B.Cu) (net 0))
 (segment (start 156.972 101.346) (end 133.35 101.346) (width 0.25) (layer B.Cu) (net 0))
 (segment (start 165.1 112.014) (end 159.004 105.918) (width 0.25) (layer F.Cu) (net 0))
 (segment (start 157.988 104.902) (end 159.004 105.918) (width 0.25) (layer B.Cu) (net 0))
 (segment (start 157.48 107.442) (end 157.48 101.854) (width 0.25) (layer F.Cu) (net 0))
 (segment (start 161.29 111.252) (end 157.48 107.442) (width 0.25) (layer F.Cu) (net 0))
 (segment (start 161.29 118.11) (end 161.29 111.252) (width 0.25) (layer F.Cu) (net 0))
 (segment (start 156.972 101.346) (end 157.48 101.854) (width 0.25) (layer B.Cu) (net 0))
 (segment (start 156.21 63.5) (end 156.21 94.996) (width 0.25) (layer B.Cu) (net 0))
 (segment (start 152.654 98.552) (end 133.096 98.552) (width 0.25) (layer B.Cu) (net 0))
 (segment (start 156.21 94.996) (end 152.654 98.552) (width 0.25) (layer B.Cu) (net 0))
 (segment (start 135.89 58.42) (end 145.288 58.42) (width 0.25) (layer B.Cu) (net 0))
 (segment (start 145.288 58.42) (end 154.686 67.818) (width 0.25) (layer B.Cu) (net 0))
 (segment (start 154.686 67.818) (end 154.686 93.472) (width 0.25) (layer B.Cu) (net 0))
 (segment (start 152.146 96.012) (end 133.096 96.012) (width 0.25) (layer B.Cu) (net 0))
 (segment (start 154.686 93.472) (end 152.146 96.012) (width 0.25) (layer B.Cu) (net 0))
 (segment (start 135.89 55.88) (end 128.016 55.88) (width 0.25) (layer B.Cu) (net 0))
 (segment (start 128.016 55.88) (end 123.952 59.944) (width 0.25) (layer B.Cu) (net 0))
 (segment (start 123.952 59.944) (end 123.952 94.996) (width 0.25) (layer B.Cu) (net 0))
 (segment (start 124.968 96.012) (end 130.556 96.012) (width 0.25) (layer B.Cu) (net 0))
 (segment (start 123.952 94.996) (end 124.968 96.012) (width 0.25) (layer B.Cu) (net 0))
 (segment (start 130.556 93.472) (end 130.556 91.186) (width 0.25) (layer F.Cu) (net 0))
 (segment (start 130.556 91.186) (end 132.334 89.408) (width 0.25) (layer F.Cu) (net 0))
 (segment (start 132.334 89.408) (end 147.828 89.408) (width 0.25) (layer F.Cu) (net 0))
 (segment (start 147.828 89.408) (end 157.099 98.679) (width 0.25) (layer F.Cu) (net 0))
 (segment (start 157.099 98.679) (end 157.226 98.552) (width 0.25) (layer F.Cu) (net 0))
 (segment (start 156.21 99.568) (end 157.099 98.679) (width 0.25) (layer F.Cu) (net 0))
 (segment (start 135.89 60.96) (end 134.366 60.96) (width 0.25) (layer B.Cu) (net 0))
 (segment (start 133.096 62.23) (end 133.096 93.472) (width 0.25) (layer B.Cu) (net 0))
 (segment (start 134.366 60.96) (end 133.096 62.23) (width 0.25) (layer B.Cu) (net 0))
 (segment (start 130.556 106.172) (end 130.556 103.632) (width 0.25) (layer F.Cu) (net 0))
 (segment (start 151.638 106.172) (end 130.556 106.172) (width 0.25) (layer F.Cu) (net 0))
 (segment (start 156.21 110.744) (end 151.638 106.172) (width 0.25) (layer F.Cu) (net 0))
 (segment (start 156.21 108.966) (end 156.21 110.744) (width 0.25) (layer F.Cu) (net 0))
 (segment (start 201.168 104.394) (end 191.77 113.792) (width 0.25) (layer B.Cu) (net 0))
 (segment (start 222.504 104.394) (end 201.168 104.394) (width 0.25) (layer B.Cu) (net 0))
 (segment (start 223.774 103.124) (end 222.504 104.394) (width 0.25) (layer B.Cu) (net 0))
 (segment (start 186.944 113.792) (end 191.77 113.792) (width 0.25) (layer B.Cu) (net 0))
 (segment (start 204.47 118.11) (end 204.47 119.888) (width 0.25) (layer B.Cu) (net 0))
 (segment (start 204.47 119.888) (end 206.248 121.666) (width 0.25) (layer B.Cu) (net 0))
 (segment (start 206.248 121.666) (end 233.426 121.666) (width 0.25) (layer B.Cu) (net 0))
 (segment (start 233.426 121.666) (end 239.776 115.316) (width 0.25) (layer B.Cu) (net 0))
 (segment (start 239.776 107.95) (end 234.696 102.87) (width 0.25) (layer B.Cu) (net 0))
 (segment (start 239.776 115.316) (end 239.776 107.95) (width 0.25) (layer B.Cu) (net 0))
 (segment (start 184.15 120.904) (end 184.15 118.11) (width 0.25) (layer B.Cu) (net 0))
 (segment (start 167.64 120.904) (end 184.15 120.904) (width 0.25) (layer B.Cu) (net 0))
 (segment (start 188.976 118.364) (end 189.23 118.11) (width 0.25) (layer B.Cu) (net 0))
 (segment (start 188.976 120.904) (end 188.976 118.364) (width 0.25) (layer B.Cu) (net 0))
 (segment (start 184.15 120.904) (end 188.976 120.904) (width 0.25) (layer B.Cu) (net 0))
 (segment (start 186.944 117.856) (end 186.69 118.11) (width 0.25) (layer B.Cu) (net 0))
 (segment (start 186.944 113.792) (end 186.944 117.856) (width 0.25) (layer B.Cu) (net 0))
 (segment (start 196.85 110.49) (end 189.23 118.11) (width 0.25) (layer B.Cu) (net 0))
 (segment (start 224.028 110.49) (end 196.85 110.49) (width 0.25) (layer B.Cu) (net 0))
 (segment (start 230.124 104.394) (end 224.028 110.49) (width 0.25) (layer B.Cu) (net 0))
 (via (at 199.644 108.966) (size 0.8) (drill 0.4) (layers F.Cu B.Cu) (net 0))
 (via (at 199.39 112.522) (size 0.8) (drill 0.4) (layers F.Cu B.Cu) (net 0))
 (segment (start 201.93 106.68) (end 199.644 108.966) (width 0.25) (layer B.Cu) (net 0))
 (segment (start 201.93 106.172) (end 201.93 106.68) (width 0.25) (layer B.Cu) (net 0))
 (segment (start 197.358 112.522) (end 191.77 118.11) (width 0.25) (layer B.Cu) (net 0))
 (segment (start 199.39 112.522) (end 197.358 112.522) (width 0.25) (layer B.Cu) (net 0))
 (segment (start 199.39 109.22) (end 199.644 108.966) (width 0.25) (layer F.Cu) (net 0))
 (segment (start 199.39 112.522) (end 199.39 109.22) (width 0.25) (layer F.Cu) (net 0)))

